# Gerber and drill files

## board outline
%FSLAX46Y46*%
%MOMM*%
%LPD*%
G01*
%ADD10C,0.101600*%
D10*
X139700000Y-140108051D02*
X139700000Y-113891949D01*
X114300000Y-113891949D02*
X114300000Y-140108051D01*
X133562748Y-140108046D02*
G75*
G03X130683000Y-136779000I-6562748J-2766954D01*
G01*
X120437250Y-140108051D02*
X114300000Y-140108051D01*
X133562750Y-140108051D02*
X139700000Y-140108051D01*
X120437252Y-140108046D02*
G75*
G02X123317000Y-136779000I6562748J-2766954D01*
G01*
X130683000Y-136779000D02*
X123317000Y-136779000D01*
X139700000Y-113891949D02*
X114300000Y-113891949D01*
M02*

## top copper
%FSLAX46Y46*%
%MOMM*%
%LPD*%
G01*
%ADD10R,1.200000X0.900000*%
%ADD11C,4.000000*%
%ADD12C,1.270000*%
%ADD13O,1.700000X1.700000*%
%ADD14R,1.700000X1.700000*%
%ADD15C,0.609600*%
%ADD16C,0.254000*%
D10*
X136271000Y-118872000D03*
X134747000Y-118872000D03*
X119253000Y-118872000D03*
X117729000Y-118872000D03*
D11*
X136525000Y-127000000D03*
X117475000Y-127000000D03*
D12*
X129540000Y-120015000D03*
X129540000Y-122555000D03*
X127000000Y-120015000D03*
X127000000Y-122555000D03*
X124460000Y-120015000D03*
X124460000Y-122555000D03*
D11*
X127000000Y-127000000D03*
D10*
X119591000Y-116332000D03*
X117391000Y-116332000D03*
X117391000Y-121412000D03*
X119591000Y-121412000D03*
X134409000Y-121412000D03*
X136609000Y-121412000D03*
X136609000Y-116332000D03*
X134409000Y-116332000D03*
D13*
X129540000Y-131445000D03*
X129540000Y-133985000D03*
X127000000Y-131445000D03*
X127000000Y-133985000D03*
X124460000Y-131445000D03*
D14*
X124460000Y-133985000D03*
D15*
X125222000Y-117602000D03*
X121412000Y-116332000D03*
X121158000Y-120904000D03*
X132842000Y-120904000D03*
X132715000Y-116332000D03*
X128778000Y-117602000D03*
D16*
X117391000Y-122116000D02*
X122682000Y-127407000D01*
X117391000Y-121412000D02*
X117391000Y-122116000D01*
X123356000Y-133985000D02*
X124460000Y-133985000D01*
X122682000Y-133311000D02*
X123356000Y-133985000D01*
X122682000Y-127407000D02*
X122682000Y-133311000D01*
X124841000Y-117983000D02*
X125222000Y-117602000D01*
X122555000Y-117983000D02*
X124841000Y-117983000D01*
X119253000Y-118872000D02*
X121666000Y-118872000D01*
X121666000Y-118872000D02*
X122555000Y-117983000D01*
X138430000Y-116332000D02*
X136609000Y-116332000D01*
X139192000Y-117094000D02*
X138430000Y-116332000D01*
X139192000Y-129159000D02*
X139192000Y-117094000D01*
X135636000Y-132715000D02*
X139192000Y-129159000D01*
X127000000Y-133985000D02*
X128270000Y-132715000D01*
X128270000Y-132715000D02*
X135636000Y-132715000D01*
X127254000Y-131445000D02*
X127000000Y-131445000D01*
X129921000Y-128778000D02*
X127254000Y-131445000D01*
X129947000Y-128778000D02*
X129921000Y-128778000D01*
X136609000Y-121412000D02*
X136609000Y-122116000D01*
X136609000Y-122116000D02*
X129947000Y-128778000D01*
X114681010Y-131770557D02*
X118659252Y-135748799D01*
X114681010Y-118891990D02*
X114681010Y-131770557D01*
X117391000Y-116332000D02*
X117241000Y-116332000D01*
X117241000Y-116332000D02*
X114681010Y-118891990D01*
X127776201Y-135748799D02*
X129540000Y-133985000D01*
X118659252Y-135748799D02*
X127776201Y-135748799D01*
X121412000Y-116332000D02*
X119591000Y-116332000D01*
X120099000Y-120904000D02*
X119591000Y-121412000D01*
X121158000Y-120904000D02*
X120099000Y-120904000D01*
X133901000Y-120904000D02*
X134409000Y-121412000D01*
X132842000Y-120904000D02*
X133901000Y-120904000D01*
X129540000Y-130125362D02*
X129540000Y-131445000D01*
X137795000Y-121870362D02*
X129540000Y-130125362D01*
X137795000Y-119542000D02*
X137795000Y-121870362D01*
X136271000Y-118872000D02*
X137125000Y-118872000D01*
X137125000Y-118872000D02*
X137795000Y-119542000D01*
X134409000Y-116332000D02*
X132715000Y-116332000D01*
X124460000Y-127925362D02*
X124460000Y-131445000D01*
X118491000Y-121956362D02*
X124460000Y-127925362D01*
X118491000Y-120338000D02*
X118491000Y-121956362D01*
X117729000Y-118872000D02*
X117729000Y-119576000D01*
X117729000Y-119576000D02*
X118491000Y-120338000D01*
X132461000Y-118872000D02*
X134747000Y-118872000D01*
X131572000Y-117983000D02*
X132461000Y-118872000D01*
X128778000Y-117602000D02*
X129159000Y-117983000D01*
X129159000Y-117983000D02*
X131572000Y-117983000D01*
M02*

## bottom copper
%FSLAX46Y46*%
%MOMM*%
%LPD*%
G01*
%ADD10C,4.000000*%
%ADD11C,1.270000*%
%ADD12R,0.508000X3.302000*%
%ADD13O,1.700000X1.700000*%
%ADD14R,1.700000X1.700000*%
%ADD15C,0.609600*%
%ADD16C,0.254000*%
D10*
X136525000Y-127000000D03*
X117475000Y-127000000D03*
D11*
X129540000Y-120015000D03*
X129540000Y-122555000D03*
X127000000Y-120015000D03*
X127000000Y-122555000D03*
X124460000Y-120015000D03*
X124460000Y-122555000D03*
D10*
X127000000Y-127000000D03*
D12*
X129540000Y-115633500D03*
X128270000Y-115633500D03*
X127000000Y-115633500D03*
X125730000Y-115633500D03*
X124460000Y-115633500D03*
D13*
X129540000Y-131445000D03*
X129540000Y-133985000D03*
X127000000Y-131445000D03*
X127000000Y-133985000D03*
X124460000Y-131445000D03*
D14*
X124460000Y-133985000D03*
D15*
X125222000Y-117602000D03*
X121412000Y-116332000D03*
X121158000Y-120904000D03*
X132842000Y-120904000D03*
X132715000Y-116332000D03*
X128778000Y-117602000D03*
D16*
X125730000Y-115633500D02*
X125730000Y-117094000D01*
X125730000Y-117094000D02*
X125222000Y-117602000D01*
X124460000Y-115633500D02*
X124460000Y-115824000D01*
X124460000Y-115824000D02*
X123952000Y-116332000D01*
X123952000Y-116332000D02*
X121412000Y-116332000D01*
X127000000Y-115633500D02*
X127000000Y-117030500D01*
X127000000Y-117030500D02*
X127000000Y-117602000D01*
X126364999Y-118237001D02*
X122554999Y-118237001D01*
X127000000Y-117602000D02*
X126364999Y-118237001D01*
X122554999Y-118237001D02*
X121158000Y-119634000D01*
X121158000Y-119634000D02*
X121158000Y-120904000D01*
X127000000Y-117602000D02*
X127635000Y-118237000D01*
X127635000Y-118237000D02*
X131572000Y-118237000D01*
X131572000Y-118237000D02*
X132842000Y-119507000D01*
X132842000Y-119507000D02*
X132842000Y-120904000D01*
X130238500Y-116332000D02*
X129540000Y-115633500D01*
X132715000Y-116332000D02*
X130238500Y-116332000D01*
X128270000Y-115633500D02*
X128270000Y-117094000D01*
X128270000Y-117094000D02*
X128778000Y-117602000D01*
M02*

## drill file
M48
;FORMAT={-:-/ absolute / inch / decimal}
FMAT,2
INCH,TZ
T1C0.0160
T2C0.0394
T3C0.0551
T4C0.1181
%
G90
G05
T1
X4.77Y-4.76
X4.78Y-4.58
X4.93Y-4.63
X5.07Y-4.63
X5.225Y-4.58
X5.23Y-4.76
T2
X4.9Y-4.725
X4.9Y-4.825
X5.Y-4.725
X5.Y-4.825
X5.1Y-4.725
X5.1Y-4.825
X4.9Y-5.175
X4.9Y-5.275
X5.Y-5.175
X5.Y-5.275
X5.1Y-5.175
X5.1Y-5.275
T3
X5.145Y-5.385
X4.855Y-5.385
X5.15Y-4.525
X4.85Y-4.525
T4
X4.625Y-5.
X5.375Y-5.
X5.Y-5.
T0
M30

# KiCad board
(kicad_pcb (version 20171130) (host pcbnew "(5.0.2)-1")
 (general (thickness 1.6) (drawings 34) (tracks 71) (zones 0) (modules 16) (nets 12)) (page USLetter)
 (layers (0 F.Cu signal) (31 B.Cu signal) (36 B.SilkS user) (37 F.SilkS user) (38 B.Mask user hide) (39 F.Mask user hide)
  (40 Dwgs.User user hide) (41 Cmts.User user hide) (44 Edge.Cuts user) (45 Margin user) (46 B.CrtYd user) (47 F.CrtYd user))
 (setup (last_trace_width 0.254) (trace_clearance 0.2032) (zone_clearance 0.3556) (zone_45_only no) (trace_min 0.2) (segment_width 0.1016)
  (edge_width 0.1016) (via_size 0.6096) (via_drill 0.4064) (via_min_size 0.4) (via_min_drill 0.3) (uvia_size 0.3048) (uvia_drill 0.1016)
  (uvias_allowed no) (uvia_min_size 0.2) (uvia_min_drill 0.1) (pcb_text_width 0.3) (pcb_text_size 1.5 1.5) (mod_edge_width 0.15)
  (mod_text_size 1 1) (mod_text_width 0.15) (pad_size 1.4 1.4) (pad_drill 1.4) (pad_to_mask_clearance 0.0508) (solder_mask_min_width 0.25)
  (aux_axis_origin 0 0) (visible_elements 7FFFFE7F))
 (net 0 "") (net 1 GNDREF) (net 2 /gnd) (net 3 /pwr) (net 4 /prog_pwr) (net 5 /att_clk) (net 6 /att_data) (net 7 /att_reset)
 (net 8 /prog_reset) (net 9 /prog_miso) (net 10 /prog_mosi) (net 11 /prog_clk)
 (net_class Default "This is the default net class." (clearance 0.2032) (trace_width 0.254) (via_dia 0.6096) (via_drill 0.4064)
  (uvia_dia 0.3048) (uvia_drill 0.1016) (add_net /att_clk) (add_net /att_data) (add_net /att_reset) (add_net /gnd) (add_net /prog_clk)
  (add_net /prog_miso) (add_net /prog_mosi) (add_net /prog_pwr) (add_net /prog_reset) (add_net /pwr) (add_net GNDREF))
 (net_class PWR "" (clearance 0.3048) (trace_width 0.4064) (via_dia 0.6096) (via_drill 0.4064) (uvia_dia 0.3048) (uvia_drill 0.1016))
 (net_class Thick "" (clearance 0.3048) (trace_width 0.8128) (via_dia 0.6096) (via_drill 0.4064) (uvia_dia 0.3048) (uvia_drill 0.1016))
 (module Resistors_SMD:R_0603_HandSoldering (layer F.Cu) (at 135.509 118.872)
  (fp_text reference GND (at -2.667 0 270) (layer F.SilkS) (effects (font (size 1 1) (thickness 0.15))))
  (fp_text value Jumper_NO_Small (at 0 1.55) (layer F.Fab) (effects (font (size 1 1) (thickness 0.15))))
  (pad 2 smd rect (at 0.762 0) (size 1.2 0.9) (layers F.Cu F.Paste F.Mask) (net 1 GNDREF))
  (pad 1 smd rect (at -0.762 0) (size 1.2 0.9) (layers F.Cu F.Paste F.Mask) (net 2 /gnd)))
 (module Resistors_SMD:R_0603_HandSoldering (layer F.Cu) (at 118.491 118.872 180)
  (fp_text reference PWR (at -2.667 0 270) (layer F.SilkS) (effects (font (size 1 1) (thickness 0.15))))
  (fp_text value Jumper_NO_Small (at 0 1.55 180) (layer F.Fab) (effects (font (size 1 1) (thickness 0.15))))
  (pad 1 smd rect (at -0.762 0 180) (size 1.2 0.9) (layers F.Cu F.Paste F.Mask) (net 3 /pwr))
  (pad 2 smd rect (at 0.762 0 180) (size 1.2 0.9) (layers F.Cu F.Paste F.Mask) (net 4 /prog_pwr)))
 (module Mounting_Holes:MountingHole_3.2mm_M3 (layer F.Cu) (at 145.415 131.5085)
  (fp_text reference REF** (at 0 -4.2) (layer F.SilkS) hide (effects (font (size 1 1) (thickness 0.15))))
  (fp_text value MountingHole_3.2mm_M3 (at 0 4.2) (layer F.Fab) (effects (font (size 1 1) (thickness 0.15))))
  (pad "" np_thru_hole circle (at -14.732 5.2705) (size 1.4 1.4) (drill 1.4) (layers *.Cu *.Mask)))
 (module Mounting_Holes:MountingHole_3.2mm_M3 (layer F.Cu) (at 148.59 131.2545)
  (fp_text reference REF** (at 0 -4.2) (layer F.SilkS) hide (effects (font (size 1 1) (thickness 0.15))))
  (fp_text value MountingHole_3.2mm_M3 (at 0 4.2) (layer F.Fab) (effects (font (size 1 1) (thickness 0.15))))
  (pad "" np_thru_hole circle (at -25.273 5.5245) (size 1.4 1.4) (drill 1.4) (layers *.Cu *.Mask)))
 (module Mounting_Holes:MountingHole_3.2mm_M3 (layer F.Cu) (at 151.765 116.459)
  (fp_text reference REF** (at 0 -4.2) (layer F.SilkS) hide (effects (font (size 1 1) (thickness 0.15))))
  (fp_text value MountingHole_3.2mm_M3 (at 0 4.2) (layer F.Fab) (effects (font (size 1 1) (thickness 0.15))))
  (pad "" np_thru_hole circle (at -15.24 10.541) (size 4 4) (drill 3) (layers *.Cu *.Mask)))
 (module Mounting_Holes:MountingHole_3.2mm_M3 (layer F.Cu) (at 125.349 116.84)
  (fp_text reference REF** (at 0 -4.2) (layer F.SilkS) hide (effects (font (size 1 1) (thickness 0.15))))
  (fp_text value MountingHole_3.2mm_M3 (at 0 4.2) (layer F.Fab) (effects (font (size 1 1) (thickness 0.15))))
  (pad "" np_thru_hole circle (at -7.874 10.16) (size 4 4) (drill 3) (layers *.Cu *.Mask)))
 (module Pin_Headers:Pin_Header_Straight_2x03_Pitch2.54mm (layer F.Cu) (at 129.54 120.015 270)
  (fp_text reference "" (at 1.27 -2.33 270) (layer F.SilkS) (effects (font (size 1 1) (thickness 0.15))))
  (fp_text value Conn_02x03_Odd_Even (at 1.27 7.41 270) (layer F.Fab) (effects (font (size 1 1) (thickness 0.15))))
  (pad 1 thru_hole circle (at 0 0 270) (size 1.27 1.27) (drill 1) (layers *.Cu *.Mask))
  (pad 2 thru_hole circle (at 2.54 0 270) (size 1.27 1.27) (drill 1) (layers *.Cu *.Mask))
  (pad 3 thru_hole circle (at 0 2.54 270) (size 1.27 1.27) (drill 1) (layers *.Cu *.Mask))
  (pad 4 thru_hole circle (at 2.54 2.54 270) (size 1.27 1.27) (drill 1) (layers *.Cu *.Mask))
  (pad 5 thru_hole circle (at 0 5.08 270) (size 1.27 1.27) (drill 1) (layers *.Cu *.Mask))
  (pad 6 thru_hole circle (at 2.54 5.08 270) (size 1.27 1.27) (drill 1) (layers *.Cu *.Mask)))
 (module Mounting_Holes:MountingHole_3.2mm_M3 (layer F.Cu) (at 128.27 116.84)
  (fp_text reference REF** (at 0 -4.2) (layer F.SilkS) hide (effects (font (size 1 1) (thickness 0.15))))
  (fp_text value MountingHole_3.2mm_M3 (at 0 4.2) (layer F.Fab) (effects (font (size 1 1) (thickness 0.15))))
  (pad "" np_thru_hole circle (at -1.27 10.16) (size 4 4) (drill 3) (layers *.Cu *.Mask)))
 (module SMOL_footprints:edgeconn (layer B.Cu) (at 124.46 115.6335 270)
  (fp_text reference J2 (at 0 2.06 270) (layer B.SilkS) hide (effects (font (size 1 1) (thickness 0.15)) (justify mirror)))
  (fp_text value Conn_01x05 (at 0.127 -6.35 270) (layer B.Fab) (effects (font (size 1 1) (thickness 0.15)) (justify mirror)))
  (pad 5 smd rect (at 0 -5.08 270) (size 3.302 0.508) (layers B.Cu B.Paste B.Mask) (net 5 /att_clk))
  (pad 4 smd rect (at 0 -3.81 270) (size 3.302 0.508) (layers B.Cu B.Paste B.Mask) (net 2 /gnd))
  (pad 3 smd rect (at 0 -2.54 270) (size 3.302 0.508) (layers B.Cu B.Paste B.Mask) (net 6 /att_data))
  (pad 2 smd rect (at 0 -1.27 270) (size 3.302 0.508) (layers B.Cu B.Paste B.Mask) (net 3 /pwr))
  (pad 1 smd rect (at 0 0 270) (size 3.302 0.508) (layers B.Cu B.Paste B.Mask) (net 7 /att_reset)))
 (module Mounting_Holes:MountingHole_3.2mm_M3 (layer F.Cu) (at 132.08 107.95)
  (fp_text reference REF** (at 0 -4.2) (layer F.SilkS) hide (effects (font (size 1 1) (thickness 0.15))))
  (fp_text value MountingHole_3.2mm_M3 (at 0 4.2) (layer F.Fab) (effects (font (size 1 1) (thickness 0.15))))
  (pad "" np_thru_hole circle (at -1.27 6.985) (size 1.4 1.4) (drill 1.4) (layers *.Cu *.Mask)))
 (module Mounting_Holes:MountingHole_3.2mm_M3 (layer F.Cu) (at 124.841 108.0135)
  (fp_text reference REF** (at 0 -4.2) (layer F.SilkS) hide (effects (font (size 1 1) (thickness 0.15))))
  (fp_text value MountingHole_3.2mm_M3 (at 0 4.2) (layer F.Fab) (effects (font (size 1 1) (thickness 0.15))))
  (pad "" np_thru_hole circle (at -1.651 6.9215) (size 1.4 1.4) (drill 1.4) (layers *.Cu *.Mask)))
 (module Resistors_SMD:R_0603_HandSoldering (layer F.Cu) (at 118.491 116.332)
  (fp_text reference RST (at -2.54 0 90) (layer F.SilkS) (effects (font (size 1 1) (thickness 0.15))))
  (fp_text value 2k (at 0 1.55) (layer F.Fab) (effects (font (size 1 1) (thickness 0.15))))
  (pad 2 smd rect (at 1.1 0) (size 1.2 0.9) (layers F.Cu F.Paste F.Mask) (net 7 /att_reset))
  (pad 1 smd rect (at -1.1 0) (size 1.2 0.9) (layers F.Cu F.Paste F.Mask) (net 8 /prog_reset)))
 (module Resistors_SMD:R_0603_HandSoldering (layer F.Cu) (at 118.491 121.412)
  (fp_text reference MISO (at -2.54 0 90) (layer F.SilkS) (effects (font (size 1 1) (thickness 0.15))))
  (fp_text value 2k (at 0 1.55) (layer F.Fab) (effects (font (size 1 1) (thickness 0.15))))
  (pad 1 smd rect (at -1.1 0) (size 1.2 0.9) (layers F.Cu F.Paste F.Mask) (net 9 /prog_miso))
  (pad 2 smd rect (at 1.1 0) (size 1.2 0.9) (layers F.Cu F.Paste F.Mask) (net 6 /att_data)))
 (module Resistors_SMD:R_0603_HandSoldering (layer F.Cu) (at 135.509 121.412 180)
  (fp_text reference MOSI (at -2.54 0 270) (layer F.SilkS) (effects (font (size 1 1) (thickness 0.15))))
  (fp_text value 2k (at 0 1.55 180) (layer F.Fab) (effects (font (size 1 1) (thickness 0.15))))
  (pad 2 smd rect (at 1.1 0 180) (size 1.2 0.9) (layers F.Cu F.Paste F.Mask) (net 6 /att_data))
  (pad 1 smd rect (at -1.1 0 180) (size 1.2 0.9) (layers F.Cu F.Paste F.Mask) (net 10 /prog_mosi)))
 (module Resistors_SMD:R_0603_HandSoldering (layer F.Cu) (at 135.509 116.332 180)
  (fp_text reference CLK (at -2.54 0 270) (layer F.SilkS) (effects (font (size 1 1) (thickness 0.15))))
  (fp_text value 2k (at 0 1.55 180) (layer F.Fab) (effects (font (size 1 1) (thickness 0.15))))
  (pad 1 smd rect (at -1.1 0 180) (size 1.2 0.9) (layers F.Cu F.Paste F.Mask) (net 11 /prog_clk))
  (pad 2 smd rect (at 1.1 0 180) (size 1.2 0.9) (layers F.Cu F.Paste F.Mask) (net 5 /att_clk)))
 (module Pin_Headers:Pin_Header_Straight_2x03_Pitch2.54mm (layer F.Cu) (at 124.46 133.985 90)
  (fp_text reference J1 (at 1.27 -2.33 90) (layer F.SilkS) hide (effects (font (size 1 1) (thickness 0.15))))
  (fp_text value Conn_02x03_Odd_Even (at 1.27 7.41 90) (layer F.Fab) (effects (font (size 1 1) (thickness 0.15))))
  (pad 6 thru_hole oval (at 2.54 5.08 90) (size 1.7 1.7) (drill 1) (layers *.Cu *.Mask) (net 1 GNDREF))
  (pad 5 thru_hole oval (at 0 5.08 90) (size 1.7 1.7) (drill 1) (layers *.Cu *.Mask) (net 8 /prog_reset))
  (pad 4 thru_hole oval (at 2.54 2.54 90) (size 1.7 1.7) (drill 1) (layers *.Cu *.Mask) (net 10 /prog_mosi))
  (pad 3 thru_hole oval (at 0 2.54 90) (size 1.7 1.7) (drill 1) (layers *.Cu *.Mask) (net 11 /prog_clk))
  (pad 2 thru_hole oval (at 2.54 0 90) (size 1.7 1.7) (drill 1) (layers *.Cu *.Mask) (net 4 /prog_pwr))
  (pad 1 thru_hole rect (at 0 0 90) (size 1.7 1.7) (drill 1) (layers *.Cu *.Mask) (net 9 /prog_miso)))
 (gr_line (start 139.7 140.108051) (end 139.7 113.891949) (layer Edge.Cuts) (width 0.1016))
 (gr_line (start 114.3 113.891949) (end 114.3 140.108051) (layer Edge.Cuts) (width 0.1016))
 (gr_arc (start 127 142.875) (end 130.683 136.779) (angle 36) (layer Edge.Cuts) (width 0.1016))
 (gr_line (start 120.43725 140.108051) (end 114.3 140.108051) (layer Edge.Cuts) (width 0.1016))
 (gr_line (start 133.56275 140.108051) (end 139.7 140.108051) (layer Edge.Cuts) (width 0.1016))
 (gr_arc (start 127 142.875) (end 123.317 136.779) (angle -36) (layer Edge.Cuts) (width 0.1016))
 (gr_line (start 130.683 136.779) (end 123.317 136.779) (layer Edge.Cuts) (width 0.1016))
 (gr_line (start 139.7 113.891949) (end 114.3 113.891949) (layer Edge.Cuts) (width 0.1016))
 (segment (start 117.391 122.116) (end 122.682 127.407) (width 0.254) (layer F.Cu) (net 9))
 (segment (start 117.391 121.412) (end 117.391 122.116) (width 0.254) (layer F.Cu) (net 9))
 (segment (start 123.356 133.985) (end 124.46 133.985) (width 0.254) (layer F.Cu) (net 9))
 (segment (start 122.682 133.311) (end 123.356 133.985) (width 0.254) (layer F.Cu) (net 9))
 (segment (start 122.682 127.407) (end 122.682 133.311) (width 0.254) (layer F.Cu) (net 9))
 (via (at 125.222 117.602) (size 0.6096) (drill 0.4064) (layers F.Cu B.Cu) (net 3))
 (segment (start 125.73 115.6335) (end 125.73 117.094) (width 0.254) (layer B.Cu) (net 3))
 (segment (start 125.73 117.094) (end 125.222 117.602) (width 0.254) (layer B.Cu) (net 3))
 (segment (start 124.841 117.983) (end 125.222 117.602) (width 0.254) (layer F.Cu) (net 3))
 (segment (start 122.555 117.983) (end 124.841 117.983) (width 0.254) (layer F.Cu) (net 3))
 (segment (start 119.253 118.872) (end 121.666 118.872) (width 0.254) (layer F.Cu) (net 3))
 (segment (start 121.666 118.872) (end 122.555 117.983) (width 0.254) (layer F.Cu) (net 3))
 (segment (start 138.43 116.332) (end 136.609 116.332) (width 0.254) (layer F.Cu) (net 11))
 (segment (start 139.192 117.094) (end 138.43 116.332) (width 0.254) (layer F.Cu) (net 11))
 (segment (start 139.192 129.159) (end 139.192 117.094) (width 0.254) (layer F.Cu) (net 11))
 (segment (start 135.636 132.715) (end 139.192 129.159) (width 0.254) (layer F.Cu) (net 11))
 (segment (start 127 133.985) (end 128.27 132.715) (width 0.254) (layer F.Cu) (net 11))
 (segment (start 128.27 132.715) (end 135.636 132.715) (width 0.254) (layer F.Cu) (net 11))
 (segment (start 127.254 131.445) (end 127 131.445) (width 0.254) (layer F.Cu) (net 10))
 (segment (start 129.921 128.778) (end 127.254 131.445) (width 0.254) (layer F.Cu) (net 10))
 (segment (start 129.947 128.778) (end 129.921 128.778) (width 0.254) (layer F.Cu) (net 10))
 (segment (start 136.609 121.412) (end 136.609 122.116) (width 0.254) (layer F.Cu) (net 10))
 (segment (start 136.609 122.116) (end 129.947 128.778) (width 0.254) (layer F.Cu) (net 10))
 (segment (start 114.68101 131.770557) (end 118.659252 135.748799) (width 0.254) (layer F.Cu) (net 8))
 (segment (start 114.68101 118.89199) (end 114.68101 131.770557) (width 0.254) (layer F.Cu) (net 8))
 (segment (start 117.391 116.332) (end 117.241 116.332) (width 0.254) (layer F.Cu) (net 8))
 (segment (start 117.241 116.332) (end 114.68101 118.89199) (width 0.254) (layer F.Cu) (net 8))
 (segment (start 127.776201 135.748799) (end 129.54 133.985) (width 0.254) (layer F.Cu) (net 8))
 (segment (start 118.659252 135.748799) (end 127.776201 135.748799) (width 0.254) (layer F.Cu) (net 8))
 (segment (start 124.46 115.6335) (end 124.46 115.824) (width 0.254) (layer B.Cu) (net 7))
 (via (at 121.412 116.332) (size 0.6096) (drill 0.4064) (layers F.Cu B.Cu) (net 7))
 (segment (start 124.46 115.824) (end 123.952 116.332) (width 0.254) (layer B.Cu) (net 7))
 (segment (start 123.952 116.332) (end 121.412 116.332) (width 0.254) (layer B.Cu) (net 7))
 (segment (start 121.412 116.332) (end 119.591 116.332) (width 0.254) (layer F.Cu) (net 7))
 (segment (start 127 115.6335) (end 127 117.0305) (width 0.254) (layer B.Cu) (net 6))
 (segment (start 127 117.0305) (end 127 117.602) (width 0.254) (layer B.Cu) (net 6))
 (segment (start 126.364999 118.237001) (end 122.554999 118.237001) (width 0.254) (layer B.Cu) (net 6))
 (segment (start 127 117.602) (end 126.364999 118.237001) (width 0.254) (layer B.Cu) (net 6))
 (via (at 121.158 120.904) (size 0.6096) (drill 0.4064) (layers F.Cu B.Cu) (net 6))
 (segment (start 122.554999 118.237001) (end 121.158 119.634) (width 0.254) (layer B.Cu) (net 6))
 (segment (start 121.158 119.634) (end 121.158 120.904) (width 0.254) (layer B.Cu) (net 6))
 (segment (start 120.099 120.904) (end 119.591 121.412) (width 0.254) (layer F.Cu) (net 6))
 (segment (start 121.158 120.904) (end 120.099 120.904) (width 0.254) (layer F.Cu) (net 6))
 (segment (start 127 117.602) (end 127.635 118.237) (width 0.254) (layer B.Cu) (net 6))
 (segment (start 127.635 118.237) (end 131.572 118.237) (width 0.254) (layer B.Cu) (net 6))
 (via (at 132.842 120.904) (size 0.6096) (drill 0.4064) (layers F.Cu B.Cu) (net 6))
 (segment (start 131.572 118.237) (end 132.842 119.507) (width 0.254) (layer B.Cu) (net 6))
 (segment (start 132.842 119.507) (end 132.842 120.904) (width 0.254) (layer B.Cu) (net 6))
 (segment (start 133.901 120.904) (end 134.409 121.412) (width 0.254) (layer F.Cu) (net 6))
 (segment (start 132.842 120.904) (end 133.901 120.904) (width 0.254) (layer F.Cu) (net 6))
 (segment (start 129.54 130.125362) (end 129.54 131.445) (width 0.254) (layer F.Cu) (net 1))
 (segment (start 137.795 121.870362) (end 129.54 130.125362) (width 0.254) (layer F.Cu) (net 1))
 (segment (start 137.795 119.542) (end 137.795 121.870362) (width 0.254) (layer F.Cu) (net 1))
 (segment (start 136.271 118.872) (end 137.125 118.872) (width 0.254) (layer F.Cu) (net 1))
 (segment (start 137.125 118.872) (end 137.795 119.542) (width 0.254) (layer F.Cu) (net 1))
 (via (at 132.715 116.332) (size 0.6096) (drill 0.4064) (layers F.Cu B.Cu) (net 5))
 (segment (start 134.409 116.332) (end 132.715 116.332) (width 0.254) (layer F.Cu) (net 5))
 (segment (start 130.2385 116.332) (end 129.54 115.6335) (width 0.254) (layer B.Cu) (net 5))
 (segment (start 132.715 116.332) (end 130.2385 116.332) (width 0.254) (layer B.Cu) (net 5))
 (segment (start 124.46 127.925362) (end 124.46 131.445) (width 0.254) (layer F.Cu) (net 4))
 (segment (start 118.491 121.956362) (end 124.46 127.925362) (width 0.254) (layer F.Cu) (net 4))
 (segment (start 118.491 120.338) (end 118.491 121.956362) (width 0.254) (layer F.Cu) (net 4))
 (segment (start 117.729 118.872) (end 117.729 119.576) (width 0.254) (layer F.Cu) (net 4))
 (segment (start 117.729 119.576) (end 118.491 120.338) (width 0.254) (layer F.Cu) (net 4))
 (via (at 128.778 117.602) (size 0.6096) (drill 0.4064) (layers F.Cu B.Cu) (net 2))
 (segment (start 128.27 115.6335) (end 128.27 117.094) (width 0.254) (layer B.Cu) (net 2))
 (segment (start 128.27 117.094) (end 128.778 117.602) (width 0.254) (layer B.Cu) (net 2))
 (segment (start 132.461 118.872) (end 134.747 118.872) (width 0.254) (layer F.Cu) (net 2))
 (segment (start 131.572 117.983) (end 132.461 118.872) (width 0.254) (layer F.Cu) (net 2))
 (segment (start 128.778 117.602) (end 129.159 117.983) (width 0.254) (layer F.Cu) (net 2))
 (segment (start 129.159 117.983) (end 131.572 117.983) (width 0.254) (layer F.Cu) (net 2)))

